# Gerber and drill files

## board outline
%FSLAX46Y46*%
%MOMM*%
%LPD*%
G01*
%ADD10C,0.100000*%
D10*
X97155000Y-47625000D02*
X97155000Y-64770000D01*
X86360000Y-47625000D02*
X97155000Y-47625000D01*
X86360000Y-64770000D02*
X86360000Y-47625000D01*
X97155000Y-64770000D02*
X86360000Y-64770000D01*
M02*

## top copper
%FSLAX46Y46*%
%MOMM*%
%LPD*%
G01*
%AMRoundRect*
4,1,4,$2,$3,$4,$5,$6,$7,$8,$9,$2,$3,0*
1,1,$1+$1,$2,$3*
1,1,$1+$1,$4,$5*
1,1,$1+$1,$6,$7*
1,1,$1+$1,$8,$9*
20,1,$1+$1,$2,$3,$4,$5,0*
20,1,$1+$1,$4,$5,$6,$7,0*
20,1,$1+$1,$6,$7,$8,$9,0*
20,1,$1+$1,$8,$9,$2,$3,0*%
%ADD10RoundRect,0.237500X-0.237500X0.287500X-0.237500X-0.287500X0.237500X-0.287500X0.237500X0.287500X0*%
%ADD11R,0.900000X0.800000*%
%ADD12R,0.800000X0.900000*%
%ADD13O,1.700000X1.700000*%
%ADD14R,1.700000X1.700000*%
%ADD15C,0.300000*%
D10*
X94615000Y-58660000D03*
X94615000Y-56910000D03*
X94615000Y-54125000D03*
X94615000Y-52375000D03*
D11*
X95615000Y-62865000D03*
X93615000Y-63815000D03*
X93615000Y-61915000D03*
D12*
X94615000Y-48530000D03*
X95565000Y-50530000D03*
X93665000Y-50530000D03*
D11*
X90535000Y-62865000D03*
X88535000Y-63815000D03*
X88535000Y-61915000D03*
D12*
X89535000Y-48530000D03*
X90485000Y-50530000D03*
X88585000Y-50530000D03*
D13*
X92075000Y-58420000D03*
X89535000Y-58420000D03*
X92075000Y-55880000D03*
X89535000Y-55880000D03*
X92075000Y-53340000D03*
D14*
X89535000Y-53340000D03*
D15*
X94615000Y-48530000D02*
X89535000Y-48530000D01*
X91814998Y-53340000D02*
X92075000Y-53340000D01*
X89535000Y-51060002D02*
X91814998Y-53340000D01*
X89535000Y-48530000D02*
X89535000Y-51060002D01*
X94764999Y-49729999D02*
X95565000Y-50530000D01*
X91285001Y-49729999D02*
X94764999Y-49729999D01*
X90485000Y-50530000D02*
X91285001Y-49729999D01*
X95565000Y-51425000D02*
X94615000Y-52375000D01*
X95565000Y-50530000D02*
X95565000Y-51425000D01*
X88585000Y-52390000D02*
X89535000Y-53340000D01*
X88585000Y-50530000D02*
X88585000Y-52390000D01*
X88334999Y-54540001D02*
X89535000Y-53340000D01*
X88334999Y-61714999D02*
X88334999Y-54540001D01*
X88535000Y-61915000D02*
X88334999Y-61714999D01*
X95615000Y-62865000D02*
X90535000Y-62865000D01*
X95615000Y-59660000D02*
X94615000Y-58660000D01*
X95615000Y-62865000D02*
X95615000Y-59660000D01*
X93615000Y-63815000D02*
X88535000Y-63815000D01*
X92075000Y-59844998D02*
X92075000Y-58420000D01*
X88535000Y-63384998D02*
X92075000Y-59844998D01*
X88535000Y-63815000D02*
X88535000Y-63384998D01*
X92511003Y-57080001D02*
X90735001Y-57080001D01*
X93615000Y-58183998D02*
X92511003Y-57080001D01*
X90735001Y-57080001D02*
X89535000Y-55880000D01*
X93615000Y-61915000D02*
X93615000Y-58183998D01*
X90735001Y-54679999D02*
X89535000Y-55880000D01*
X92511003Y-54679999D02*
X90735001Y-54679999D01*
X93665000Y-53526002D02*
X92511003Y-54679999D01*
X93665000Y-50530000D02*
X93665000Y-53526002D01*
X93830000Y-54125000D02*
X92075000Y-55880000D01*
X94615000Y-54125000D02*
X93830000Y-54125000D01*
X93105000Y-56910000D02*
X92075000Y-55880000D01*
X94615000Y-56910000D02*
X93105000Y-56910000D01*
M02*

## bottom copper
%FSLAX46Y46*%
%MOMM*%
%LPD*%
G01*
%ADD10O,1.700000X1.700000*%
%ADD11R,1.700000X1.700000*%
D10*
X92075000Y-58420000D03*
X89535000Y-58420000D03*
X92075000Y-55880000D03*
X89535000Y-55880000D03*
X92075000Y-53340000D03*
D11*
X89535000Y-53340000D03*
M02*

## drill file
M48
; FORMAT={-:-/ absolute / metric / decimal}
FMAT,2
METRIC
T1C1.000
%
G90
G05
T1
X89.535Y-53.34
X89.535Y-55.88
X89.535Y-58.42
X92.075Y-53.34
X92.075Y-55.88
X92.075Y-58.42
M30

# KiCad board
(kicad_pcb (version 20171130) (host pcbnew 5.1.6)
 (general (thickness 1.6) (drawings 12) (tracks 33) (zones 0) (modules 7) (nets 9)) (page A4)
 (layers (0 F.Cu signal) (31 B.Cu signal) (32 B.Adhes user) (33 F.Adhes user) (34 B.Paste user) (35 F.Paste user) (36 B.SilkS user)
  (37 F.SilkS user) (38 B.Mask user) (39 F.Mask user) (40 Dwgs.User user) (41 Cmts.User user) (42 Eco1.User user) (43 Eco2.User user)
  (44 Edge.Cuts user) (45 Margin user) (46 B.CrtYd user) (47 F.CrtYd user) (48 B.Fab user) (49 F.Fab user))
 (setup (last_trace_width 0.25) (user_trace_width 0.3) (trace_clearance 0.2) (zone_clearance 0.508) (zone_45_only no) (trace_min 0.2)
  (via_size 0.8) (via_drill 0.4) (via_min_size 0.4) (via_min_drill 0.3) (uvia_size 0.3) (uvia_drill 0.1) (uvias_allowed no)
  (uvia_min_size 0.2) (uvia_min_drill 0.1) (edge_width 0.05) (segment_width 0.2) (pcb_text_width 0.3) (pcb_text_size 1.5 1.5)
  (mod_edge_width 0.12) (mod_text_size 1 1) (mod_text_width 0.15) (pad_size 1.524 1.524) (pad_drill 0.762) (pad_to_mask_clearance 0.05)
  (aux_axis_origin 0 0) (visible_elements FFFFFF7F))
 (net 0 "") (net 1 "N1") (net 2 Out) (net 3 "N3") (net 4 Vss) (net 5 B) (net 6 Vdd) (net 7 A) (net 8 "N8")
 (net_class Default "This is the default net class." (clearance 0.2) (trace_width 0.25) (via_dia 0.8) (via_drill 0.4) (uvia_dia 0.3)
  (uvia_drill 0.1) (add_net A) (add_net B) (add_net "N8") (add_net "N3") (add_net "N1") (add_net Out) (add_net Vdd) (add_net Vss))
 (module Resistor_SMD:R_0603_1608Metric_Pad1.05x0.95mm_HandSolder (layer F.Cu) (at 94.615 57.785 270)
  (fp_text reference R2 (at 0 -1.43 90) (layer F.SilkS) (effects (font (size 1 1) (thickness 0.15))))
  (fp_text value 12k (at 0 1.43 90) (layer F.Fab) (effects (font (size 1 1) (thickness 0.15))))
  (pad 2 smd roundrect (at 0.875 0 270) (size 1.05 0.95) (layers F.Cu F.Paste F.Mask) (roundrect_rratio 0.25) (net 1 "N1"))
  (pad 1 smd roundrect (at -0.875 0 270) (size 1.05 0.95) (layers F.Cu F.Paste F.Mask) (roundrect_rratio 0.25) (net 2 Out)))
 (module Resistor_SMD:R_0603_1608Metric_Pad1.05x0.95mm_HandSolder (layer F.Cu) (at 94.615 53.25 270)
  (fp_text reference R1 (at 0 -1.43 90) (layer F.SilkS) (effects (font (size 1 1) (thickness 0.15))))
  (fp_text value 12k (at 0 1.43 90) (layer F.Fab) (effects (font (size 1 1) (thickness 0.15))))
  (pad 2 smd roundrect (at 0.875 0 270) (size 1.05 0.95) (layers F.Cu F.Paste F.Mask) (roundrect_rratio 0.25) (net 2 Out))
  (pad 1 smd roundrect (at -0.875 0 270) (size 1.05 0.95) (layers F.Cu F.Paste F.Mask) (roundrect_rratio 0.25) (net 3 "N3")))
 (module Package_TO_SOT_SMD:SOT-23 (layer F.Cu) (at 94.615 62.865)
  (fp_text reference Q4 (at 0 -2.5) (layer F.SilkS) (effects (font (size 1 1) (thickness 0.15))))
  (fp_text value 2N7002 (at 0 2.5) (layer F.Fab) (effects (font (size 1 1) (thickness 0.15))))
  (pad 3 smd rect (at 1 0) (size 0.9 0.8) (layers F.Cu F.Paste F.Mask) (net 1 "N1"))
  (pad 2 smd rect (at -1 0.95) (size 0.9 0.8) (layers F.Cu F.Paste F.Mask) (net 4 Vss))
  (pad 1 smd rect (at -1 -0.95) (size 0.9 0.8) (layers F.Cu F.Paste F.Mask) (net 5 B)))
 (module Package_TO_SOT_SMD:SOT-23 (layer F.Cu) (at 94.615 49.53 90)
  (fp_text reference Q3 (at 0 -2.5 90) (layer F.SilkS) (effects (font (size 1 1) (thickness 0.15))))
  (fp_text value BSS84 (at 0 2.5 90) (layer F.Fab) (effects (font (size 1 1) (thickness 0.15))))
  (pad 3 smd rect (at 1 0 90) (size 0.9 0.8) (layers F.Cu F.Paste F.Mask) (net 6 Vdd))
  (pad 2 smd rect (at -1 0.95 90) (size 0.9 0.8) (layers F.Cu F.Paste F.Mask) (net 3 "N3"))
  (pad 1 smd rect (at -1 -0.95 90) (size 0.9 0.8) (layers F.Cu F.Paste F.Mask) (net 5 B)))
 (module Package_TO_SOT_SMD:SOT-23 (layer F.Cu) (at 89.535 62.865)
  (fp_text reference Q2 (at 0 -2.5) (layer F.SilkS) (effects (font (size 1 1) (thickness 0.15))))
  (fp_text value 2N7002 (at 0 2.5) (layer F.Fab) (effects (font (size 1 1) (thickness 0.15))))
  (pad 3 smd rect (at 1 0) (size 0.9 0.8) (layers F.Cu F.Paste F.Mask) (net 1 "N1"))
  (pad 2 smd rect (at -1 0.95) (size 0.9 0.8) (layers F.Cu F.Paste F.Mask) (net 4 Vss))
  (pad 1 smd rect (at -1 -0.95) (size 0.9 0.8) (layers F.Cu F.Paste F.Mask) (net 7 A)))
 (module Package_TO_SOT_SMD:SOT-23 (layer F.Cu) (at 89.535 49.53 90)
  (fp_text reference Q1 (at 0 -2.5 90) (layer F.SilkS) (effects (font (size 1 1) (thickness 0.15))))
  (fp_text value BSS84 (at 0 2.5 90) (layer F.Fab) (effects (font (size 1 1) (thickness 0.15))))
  (pad 3 smd rect (at 1 0 90) (size 0.9 0.8) (layers F.Cu F.Paste F.Mask) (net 6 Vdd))
  (pad 2 smd rect (at -1 0.95 90) (size 0.9 0.8) (layers F.Cu F.Paste F.Mask) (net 3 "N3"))
  (pad 1 smd rect (at -1 -0.95 90) (size 0.9 0.8) (layers F.Cu F.Paste F.Mask) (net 7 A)))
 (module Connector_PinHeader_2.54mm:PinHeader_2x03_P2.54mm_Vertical (layer F.Cu) (at 89.535 53.34)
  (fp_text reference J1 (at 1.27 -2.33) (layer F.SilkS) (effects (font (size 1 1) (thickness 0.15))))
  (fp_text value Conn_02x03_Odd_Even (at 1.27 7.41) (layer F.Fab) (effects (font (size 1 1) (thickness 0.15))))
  (pad 6 thru_hole oval (at 2.54 5.08) (size 1.7 1.7) (drill 1) (layers *.Cu *.Mask) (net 4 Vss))
  (pad 5 thru_hole oval (at 0 5.08) (size 1.7 1.7) (drill 1) (layers *.Cu *.Mask) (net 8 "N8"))
  (pad 4 thru_hole oval (at 2.54 2.54) (size 1.7 1.7) (drill 1) (layers *.Cu *.Mask) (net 2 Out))
  (pad 3 thru_hole oval (at 0 2.54) (size 1.7 1.7) (drill 1) (layers *.Cu *.Mask) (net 5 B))
  (pad 2 thru_hole oval (at 2.54 0) (size 1.7 1.7) (drill 1) (layers *.Cu *.Mask) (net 6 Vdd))
  (pad 1 thru_hole rect (at 0 0) (size 1.7 1.7) (drill 1) (layers *.Cu *.Mask) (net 7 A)))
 (gr_line (start 97.155 47.625) (end 97.155 64.77) (layer Edge.Cuts) (width 0.1))
 (gr_line (start 86.36 47.625) (end 97.155 47.625) (layer Edge.Cuts) (width 0.1))
 (gr_line (start 86.36 64.77) (end 86.36 47.625) (layer Edge.Cuts) (width 0.1))
 (gr_line (start 97.155 64.77) (end 86.36 64.77) (layer Edge.Cuts) (width 0.1))
 (segment (start 94.615 48.53) (end 89.535 48.53) (width 0.3) (layer F.Cu) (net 6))
 (segment (start 91.814998 53.34) (end 92.075 53.34) (width 0.3) (layer F.Cu) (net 6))
 (segment (start 89.535 51.060002) (end 91.814998 53.34) (width 0.3) (layer F.Cu) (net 6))
 (segment (start 89.535 48.53) (end 89.535 51.060002) (width 0.3) (layer F.Cu) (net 6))
 (segment (start 94.764999 49.729999) (end 95.565 50.53) (width 0.3) (layer F.Cu) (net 3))
 (segment (start 91.285001 49.729999) (end 94.764999 49.729999) (width 0.3) (layer F.Cu) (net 3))
 (segment (start 90.485 50.53) (end 91.285001 49.729999) (width 0.3) (layer F.Cu) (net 3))
 (segment (start 95.565 51.425) (end 94.615 52.375) (width 0.3) (layer F.Cu) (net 3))
 (segment (start 95.565 50.53) (end 95.565 51.425) (width 0.3) (layer F.Cu) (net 3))
 (segment (start 88.585 52.39) (end 89.535 53.34) (width 0.3) (layer F.Cu) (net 7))
 (segment (start 88.585 50.53) (end 88.585 52.39) (width 0.3) (layer F.Cu) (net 7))
 (segment (start 88.334999 54.540001) (end 89.535 53.34) (width 0.3) (layer F.Cu) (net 7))
 (segment (start 88.334999 61.714999) (end 88.334999 54.540001) (width 0.3) (layer F.Cu) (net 7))
 (segment (start 88.535 61.915) (end 88.334999 61.714999) (width 0.3) (layer F.Cu) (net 7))
 (segment (start 95.615 62.865) (end 90.535 62.865) (width 0.3) (layer F.Cu) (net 1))
 (segment (start 95.615 59.66) (end 94.615 58.66) (width 0.3) (layer F.Cu) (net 1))
 (segment (start 95.615 62.865) (end 95.615 59.66) (width 0.3) (layer F.Cu) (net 1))
 (segment (start 93.615 63.815) (end 88.535 63.815) (width 0.3) (layer F.Cu) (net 4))
 (segment (start 92.075 59.844998) (end 92.075 58.42) (width 0.3) (layer F.Cu) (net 4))
 (segment (start 88.535 63.384998) (end 92.075 59.844998) (width 0.3) (layer F.Cu) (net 4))
 (segment (start 88.535 63.815) (end 88.535 63.384998) (width 0.3) (layer F.Cu) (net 4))
 (segment (start 92.511003 57.080001) (end 90.735001 57.080001) (width 0.3) (layer F.Cu) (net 5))
 (segment (start 93.615 58.183998) (end 92.511003 57.080001) (width 0.3) (layer F.Cu) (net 5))
 (segment (start 90.735001 57.080001) (end 89.535 55.88) (width 0.3) (layer F.Cu) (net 5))
 (segment (start 93.615 61.915) (end 93.615 58.183998) (width 0.3) (layer F.Cu) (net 5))
 (segment (start 90.735001 54.679999) (end 89.535 55.88) (width 0.3) (layer F.Cu) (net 5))
 (segment (start 92.511003 54.679999) (end 90.735001 54.679999) (width 0.3) (layer F.Cu) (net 5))
 (segment (start 93.665 53.526002) (end 92.511003 54.679999) (width 0.3) (layer F.Cu) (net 5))
 (segment (start 93.665 50.53) (end 93.665 53.526002) (width 0.3) (layer F.Cu) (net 5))
 (segment (start 93.83 54.125) (end 92.075 55.88) (width 0.3) (layer F.Cu) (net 2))
 (segment (start 94.615 54.125) (end 93.83 54.125) (width 0.3) (layer F.Cu) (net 2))
 (segment (start 93.105 56.91) (end 92.075 55.88) (width 0.3) (layer F.Cu) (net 2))
 (segment (start 94.615 56.91) (end 93.105 56.91) (width 0.3) (layer F.Cu) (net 2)))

